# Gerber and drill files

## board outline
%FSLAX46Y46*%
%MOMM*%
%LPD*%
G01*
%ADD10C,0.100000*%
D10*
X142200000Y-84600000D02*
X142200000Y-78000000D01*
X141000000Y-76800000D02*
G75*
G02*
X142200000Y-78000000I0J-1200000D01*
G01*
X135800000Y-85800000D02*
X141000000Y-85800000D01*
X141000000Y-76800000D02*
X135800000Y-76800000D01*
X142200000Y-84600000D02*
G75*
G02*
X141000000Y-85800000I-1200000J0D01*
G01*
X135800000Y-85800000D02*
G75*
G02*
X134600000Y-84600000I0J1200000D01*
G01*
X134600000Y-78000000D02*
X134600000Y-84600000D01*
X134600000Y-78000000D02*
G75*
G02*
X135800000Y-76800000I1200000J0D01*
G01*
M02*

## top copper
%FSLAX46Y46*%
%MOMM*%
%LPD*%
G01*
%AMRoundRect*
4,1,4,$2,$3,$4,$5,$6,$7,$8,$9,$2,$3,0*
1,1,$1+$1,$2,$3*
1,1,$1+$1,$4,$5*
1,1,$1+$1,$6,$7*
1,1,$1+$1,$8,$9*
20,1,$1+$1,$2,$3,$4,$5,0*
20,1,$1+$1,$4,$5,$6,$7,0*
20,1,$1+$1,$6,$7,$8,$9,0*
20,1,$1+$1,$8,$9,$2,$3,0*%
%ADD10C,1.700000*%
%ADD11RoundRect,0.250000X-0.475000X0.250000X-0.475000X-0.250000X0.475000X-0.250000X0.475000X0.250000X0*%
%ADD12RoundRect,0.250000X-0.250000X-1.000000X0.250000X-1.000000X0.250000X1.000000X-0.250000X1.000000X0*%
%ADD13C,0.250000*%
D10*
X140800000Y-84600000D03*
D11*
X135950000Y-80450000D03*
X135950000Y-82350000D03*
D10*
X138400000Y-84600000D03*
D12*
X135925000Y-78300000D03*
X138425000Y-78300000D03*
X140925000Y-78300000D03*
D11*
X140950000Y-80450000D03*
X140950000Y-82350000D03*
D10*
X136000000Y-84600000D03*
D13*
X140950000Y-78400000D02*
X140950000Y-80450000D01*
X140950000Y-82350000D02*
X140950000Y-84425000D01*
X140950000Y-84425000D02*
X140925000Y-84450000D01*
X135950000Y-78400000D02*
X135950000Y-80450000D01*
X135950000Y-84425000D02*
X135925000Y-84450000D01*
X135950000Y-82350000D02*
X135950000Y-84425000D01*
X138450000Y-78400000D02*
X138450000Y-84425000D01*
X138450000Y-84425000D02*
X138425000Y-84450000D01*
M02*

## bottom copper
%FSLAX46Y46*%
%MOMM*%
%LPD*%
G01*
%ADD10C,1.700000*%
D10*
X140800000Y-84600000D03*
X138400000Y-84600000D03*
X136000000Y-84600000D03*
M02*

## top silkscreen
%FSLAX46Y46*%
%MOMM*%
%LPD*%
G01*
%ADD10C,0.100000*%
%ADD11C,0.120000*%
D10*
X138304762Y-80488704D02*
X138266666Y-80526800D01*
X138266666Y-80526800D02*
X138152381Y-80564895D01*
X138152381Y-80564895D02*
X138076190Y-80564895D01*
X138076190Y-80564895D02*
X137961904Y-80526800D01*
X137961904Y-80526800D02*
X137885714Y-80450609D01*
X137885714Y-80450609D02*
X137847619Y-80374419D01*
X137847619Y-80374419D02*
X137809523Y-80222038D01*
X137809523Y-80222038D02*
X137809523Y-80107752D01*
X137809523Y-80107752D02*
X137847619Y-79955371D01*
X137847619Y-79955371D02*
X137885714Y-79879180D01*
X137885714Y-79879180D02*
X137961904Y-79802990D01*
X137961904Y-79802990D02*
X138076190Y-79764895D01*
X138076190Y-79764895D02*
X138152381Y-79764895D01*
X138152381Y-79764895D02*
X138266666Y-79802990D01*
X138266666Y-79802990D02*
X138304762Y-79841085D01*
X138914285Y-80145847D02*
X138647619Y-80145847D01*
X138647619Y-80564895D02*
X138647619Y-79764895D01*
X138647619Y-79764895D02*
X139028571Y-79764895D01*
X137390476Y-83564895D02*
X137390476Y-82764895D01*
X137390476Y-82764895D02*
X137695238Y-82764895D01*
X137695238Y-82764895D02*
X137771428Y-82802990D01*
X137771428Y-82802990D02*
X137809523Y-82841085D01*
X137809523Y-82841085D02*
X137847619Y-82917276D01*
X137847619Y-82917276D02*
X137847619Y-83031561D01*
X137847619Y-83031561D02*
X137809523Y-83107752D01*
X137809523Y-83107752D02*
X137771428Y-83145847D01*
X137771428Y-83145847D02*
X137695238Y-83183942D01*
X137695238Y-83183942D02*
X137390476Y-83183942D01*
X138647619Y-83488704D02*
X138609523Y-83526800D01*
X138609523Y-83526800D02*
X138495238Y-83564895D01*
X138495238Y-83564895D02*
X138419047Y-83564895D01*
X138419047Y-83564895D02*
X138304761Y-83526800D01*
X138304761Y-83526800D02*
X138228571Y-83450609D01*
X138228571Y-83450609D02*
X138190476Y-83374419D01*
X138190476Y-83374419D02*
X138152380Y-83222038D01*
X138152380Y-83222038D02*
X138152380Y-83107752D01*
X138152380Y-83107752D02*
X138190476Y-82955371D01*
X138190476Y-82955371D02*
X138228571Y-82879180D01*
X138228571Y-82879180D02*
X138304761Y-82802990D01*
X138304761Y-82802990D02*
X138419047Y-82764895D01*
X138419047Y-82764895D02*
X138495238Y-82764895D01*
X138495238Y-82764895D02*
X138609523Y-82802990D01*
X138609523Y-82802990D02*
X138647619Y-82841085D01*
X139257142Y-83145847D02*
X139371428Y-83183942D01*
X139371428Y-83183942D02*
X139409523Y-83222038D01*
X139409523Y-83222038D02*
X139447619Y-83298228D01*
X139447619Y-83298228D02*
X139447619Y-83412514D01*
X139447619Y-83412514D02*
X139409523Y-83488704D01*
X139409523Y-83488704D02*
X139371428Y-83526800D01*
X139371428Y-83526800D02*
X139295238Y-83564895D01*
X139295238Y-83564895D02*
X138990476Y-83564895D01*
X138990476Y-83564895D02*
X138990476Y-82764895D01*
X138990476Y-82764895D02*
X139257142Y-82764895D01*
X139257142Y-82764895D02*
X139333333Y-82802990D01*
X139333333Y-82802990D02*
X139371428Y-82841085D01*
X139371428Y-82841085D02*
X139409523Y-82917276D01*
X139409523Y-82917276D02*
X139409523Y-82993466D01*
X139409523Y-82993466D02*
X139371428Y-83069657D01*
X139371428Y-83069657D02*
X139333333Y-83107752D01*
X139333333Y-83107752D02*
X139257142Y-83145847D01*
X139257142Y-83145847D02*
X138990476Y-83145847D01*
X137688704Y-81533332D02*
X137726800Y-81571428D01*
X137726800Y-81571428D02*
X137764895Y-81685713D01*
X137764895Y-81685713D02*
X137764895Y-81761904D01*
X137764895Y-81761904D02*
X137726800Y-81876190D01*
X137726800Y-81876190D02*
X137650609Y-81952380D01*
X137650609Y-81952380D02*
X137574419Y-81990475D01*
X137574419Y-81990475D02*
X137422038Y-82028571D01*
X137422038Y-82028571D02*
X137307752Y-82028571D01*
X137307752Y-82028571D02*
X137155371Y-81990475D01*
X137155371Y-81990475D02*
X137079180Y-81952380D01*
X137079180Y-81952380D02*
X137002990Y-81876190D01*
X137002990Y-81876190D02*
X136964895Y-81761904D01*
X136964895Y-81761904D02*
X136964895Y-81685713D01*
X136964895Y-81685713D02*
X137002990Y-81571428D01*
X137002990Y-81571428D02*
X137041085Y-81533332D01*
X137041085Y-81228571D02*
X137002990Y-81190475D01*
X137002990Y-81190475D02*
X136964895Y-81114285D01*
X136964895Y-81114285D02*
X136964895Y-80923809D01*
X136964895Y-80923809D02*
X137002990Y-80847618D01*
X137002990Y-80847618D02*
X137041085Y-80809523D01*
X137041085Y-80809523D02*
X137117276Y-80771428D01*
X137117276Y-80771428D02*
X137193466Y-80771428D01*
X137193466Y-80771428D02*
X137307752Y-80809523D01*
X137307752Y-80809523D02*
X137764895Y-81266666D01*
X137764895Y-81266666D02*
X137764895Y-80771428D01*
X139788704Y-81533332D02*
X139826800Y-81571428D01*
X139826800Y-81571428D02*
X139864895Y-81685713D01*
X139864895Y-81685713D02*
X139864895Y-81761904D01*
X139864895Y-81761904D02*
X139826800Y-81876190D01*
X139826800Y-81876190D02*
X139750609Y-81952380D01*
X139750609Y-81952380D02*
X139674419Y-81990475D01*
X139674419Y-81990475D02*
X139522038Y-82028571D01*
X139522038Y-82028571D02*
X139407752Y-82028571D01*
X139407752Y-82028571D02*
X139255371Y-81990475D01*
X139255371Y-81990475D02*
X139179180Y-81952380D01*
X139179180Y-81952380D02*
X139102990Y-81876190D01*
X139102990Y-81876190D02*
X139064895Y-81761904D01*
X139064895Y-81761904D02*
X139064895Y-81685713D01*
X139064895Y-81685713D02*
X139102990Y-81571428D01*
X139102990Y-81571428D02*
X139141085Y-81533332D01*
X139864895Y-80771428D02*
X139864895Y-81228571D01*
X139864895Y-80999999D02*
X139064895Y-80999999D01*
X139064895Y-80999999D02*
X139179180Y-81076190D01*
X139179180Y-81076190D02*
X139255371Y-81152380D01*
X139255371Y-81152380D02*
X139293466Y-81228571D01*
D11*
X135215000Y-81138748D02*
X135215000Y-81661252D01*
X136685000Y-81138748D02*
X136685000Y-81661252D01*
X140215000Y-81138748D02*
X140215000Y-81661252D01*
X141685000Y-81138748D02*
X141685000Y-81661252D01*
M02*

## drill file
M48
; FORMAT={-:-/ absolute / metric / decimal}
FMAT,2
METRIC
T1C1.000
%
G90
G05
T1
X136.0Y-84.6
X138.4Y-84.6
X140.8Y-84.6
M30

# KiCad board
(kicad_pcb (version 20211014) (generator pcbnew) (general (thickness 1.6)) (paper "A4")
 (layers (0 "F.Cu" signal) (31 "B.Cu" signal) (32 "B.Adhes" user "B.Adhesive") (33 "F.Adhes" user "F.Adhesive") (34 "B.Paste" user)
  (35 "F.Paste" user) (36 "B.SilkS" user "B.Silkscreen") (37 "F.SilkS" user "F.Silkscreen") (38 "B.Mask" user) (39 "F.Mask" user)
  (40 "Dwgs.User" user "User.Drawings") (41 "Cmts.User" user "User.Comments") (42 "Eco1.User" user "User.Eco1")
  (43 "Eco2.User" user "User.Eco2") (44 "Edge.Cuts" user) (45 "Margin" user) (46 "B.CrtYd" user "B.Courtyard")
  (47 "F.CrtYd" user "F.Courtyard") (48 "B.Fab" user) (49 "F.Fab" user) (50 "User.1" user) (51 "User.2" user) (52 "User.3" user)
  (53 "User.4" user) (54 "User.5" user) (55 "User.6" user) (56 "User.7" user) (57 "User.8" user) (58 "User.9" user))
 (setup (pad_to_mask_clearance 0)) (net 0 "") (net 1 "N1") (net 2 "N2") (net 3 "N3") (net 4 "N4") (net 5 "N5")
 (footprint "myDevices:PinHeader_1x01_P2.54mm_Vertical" (layer "F.Cu") (at 140.8 84.6 90)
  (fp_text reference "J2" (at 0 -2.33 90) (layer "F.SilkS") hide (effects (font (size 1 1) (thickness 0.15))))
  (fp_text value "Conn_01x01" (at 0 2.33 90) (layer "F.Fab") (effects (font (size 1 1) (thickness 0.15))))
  (pad "1" thru_hole circle (at 0 0 90) (size 1.7 1.7) (drill 1) (layers *.Cu *.Mask) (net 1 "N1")))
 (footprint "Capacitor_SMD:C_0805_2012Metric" (layer "F.Cu") (at 135.95 81.4 -90)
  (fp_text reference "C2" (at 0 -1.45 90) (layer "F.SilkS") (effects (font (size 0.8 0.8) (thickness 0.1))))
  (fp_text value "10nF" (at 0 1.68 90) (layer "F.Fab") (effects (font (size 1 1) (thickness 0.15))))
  (fp_line (start -0.261252 0.735) (end 0.261252 0.735) (layer "F.SilkS") (width 0.12))
  (fp_line (start -0.261252 -0.735) (end 0.261252 -0.735) (layer "F.SilkS") (width 0.12))
  (pad "1" smd roundrect (at -0.95 0 270) (size 1 1.45) (layers "F.Cu" "F.Paste" "F.Mask") (roundrect_rratio 0.25) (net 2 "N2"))
  (pad "2" smd roundrect (at 0.95 0 270) (size 1 1.45) (layers "F.Cu" "F.Paste" "F.Mask") (roundrect_rratio 0.25) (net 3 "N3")))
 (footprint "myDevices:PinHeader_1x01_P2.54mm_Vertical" (layer "F.Cu") (at 138.4 84.6)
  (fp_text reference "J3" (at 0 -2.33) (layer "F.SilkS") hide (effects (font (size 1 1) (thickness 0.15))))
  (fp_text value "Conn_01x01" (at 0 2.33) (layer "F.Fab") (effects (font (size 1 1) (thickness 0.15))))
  (pad "1" thru_hole circle (at 0 0) (size 1.7 1.7) (drill 1) (layers *.Cu *.Mask) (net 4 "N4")))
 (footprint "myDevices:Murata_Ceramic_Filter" (layer "F.Cu") (at 135.925 78.3)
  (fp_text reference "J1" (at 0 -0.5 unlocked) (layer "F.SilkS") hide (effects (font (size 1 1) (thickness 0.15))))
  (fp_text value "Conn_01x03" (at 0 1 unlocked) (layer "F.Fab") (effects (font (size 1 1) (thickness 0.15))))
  (pad "1" smd roundrect (at 0 0) (size 1 2.5) (layers "F.Cu" "F.Paste" "F.Mask") (roundrect_rratio 0.25) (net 2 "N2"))
  (pad "2" smd roundrect (at 2.5 0) (size 1 2.5) (layers "F.Cu" "F.Paste" "F.Mask") (roundrect_rratio 0.25) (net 4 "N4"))
  (pad "3" smd roundrect (at 5 0) (size 1 2.5) (layers "F.Cu" "F.Paste" "F.Mask") (roundrect_rratio 0.25) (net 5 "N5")))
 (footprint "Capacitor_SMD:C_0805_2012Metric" (layer "F.Cu") (at 140.95 81.4 -90)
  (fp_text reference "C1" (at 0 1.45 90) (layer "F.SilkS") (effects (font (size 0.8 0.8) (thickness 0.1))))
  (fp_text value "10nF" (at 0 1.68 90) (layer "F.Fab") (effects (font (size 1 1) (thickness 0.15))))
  (fp_line (start -0.261252 0.735) (end 0.261252 0.735) (layer "F.SilkS") (width 0.12))
  (fp_line (start -0.261252 -0.735) (end 0.261252 -0.735) (layer "F.SilkS") (width 0.12))
  (pad "1" smd roundrect (at -0.95 0 270) (size 1 1.45) (layers "F.Cu" "F.Paste" "F.Mask") (roundrect_rratio 0.25) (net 5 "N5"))
  (pad "2" smd roundrect (at 0.95 0 270) (size 1 1.45) (layers "F.Cu" "F.Paste" "F.Mask") (roundrect_rratio 0.25) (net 1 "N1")))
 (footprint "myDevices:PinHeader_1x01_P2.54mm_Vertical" (layer "F.Cu") (at 136 84.6 180)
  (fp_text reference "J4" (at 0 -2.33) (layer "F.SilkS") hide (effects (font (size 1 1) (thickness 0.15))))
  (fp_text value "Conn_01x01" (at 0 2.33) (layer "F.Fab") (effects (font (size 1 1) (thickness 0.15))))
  (pad "1" thru_hole circle (at 0 0 180) (size 1.7 1.7) (drill 1) (layers *.Cu *.Mask) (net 3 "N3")))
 (gr_line (start 142.2 84.6) (end 142.2 78) (layer "Edge.Cuts") (width 0.1))
 (gr_arc (start 141 76.8) (mid 141.848528 77.151472) (end 142.2 78) (layer "Edge.Cuts") (width 0.1))
 (gr_line (start 135.8 85.8) (end 141 85.8) (layer "Edge.Cuts") (width 0.1))
 (gr_line (start 141 76.8) (end 135.8 76.8) (layer "Edge.Cuts") (width 0.1))
 (gr_arc (start 142.2 84.6) (mid 141.848528 85.448528) (end 141 85.8) (layer "Edge.Cuts") (width 0.1))
 (gr_arc (start 135.8 85.8) (mid 134.951472 85.448528) (end 134.6 84.6) (layer "Edge.Cuts") (width 0.1))
 (gr_line (start 134.6 78) (end 134.6 84.6) (layer "Edge.Cuts") (width 0.1))
 (gr_arc (start 134.6 78) (mid 134.951472 77.151472) (end 135.8 76.8) (layer "Edge.Cuts") (width 0.1))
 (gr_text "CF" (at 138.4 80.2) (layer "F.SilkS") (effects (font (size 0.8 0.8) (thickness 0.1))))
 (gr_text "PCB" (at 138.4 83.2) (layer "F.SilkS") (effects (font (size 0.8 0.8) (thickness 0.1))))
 (segment (start 140.95 78.4) (end 140.95 80.45) (width 0.25) (layer "F.Cu") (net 5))
 (segment (start 140.95 82.35) (end 140.95 84.425) (width 0.25) (layer "F.Cu") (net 1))
 (segment (start 140.95 84.425) (end 140.925 84.45) (width 0.25) (layer "F.Cu") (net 1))
 (segment (start 135.95 78.4) (end 135.95 80.45) (width 0.25) (layer "F.Cu") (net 2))
 (segment (start 135.95 84.425) (end 135.925 84.45) (width 0.25) (layer "F.Cu") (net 3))
 (segment (start 135.95 82.35) (end 135.95 84.425) (width 0.25) (layer "F.Cu") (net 3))
 (segment (start 138.45 78.4) (end 138.45 84.425) (width 0.25) (layer "F.Cu") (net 4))
 (segment (start 138.45 84.425) (end 138.425 84.45) (width 0.25) (layer "F.Cu") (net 4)))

